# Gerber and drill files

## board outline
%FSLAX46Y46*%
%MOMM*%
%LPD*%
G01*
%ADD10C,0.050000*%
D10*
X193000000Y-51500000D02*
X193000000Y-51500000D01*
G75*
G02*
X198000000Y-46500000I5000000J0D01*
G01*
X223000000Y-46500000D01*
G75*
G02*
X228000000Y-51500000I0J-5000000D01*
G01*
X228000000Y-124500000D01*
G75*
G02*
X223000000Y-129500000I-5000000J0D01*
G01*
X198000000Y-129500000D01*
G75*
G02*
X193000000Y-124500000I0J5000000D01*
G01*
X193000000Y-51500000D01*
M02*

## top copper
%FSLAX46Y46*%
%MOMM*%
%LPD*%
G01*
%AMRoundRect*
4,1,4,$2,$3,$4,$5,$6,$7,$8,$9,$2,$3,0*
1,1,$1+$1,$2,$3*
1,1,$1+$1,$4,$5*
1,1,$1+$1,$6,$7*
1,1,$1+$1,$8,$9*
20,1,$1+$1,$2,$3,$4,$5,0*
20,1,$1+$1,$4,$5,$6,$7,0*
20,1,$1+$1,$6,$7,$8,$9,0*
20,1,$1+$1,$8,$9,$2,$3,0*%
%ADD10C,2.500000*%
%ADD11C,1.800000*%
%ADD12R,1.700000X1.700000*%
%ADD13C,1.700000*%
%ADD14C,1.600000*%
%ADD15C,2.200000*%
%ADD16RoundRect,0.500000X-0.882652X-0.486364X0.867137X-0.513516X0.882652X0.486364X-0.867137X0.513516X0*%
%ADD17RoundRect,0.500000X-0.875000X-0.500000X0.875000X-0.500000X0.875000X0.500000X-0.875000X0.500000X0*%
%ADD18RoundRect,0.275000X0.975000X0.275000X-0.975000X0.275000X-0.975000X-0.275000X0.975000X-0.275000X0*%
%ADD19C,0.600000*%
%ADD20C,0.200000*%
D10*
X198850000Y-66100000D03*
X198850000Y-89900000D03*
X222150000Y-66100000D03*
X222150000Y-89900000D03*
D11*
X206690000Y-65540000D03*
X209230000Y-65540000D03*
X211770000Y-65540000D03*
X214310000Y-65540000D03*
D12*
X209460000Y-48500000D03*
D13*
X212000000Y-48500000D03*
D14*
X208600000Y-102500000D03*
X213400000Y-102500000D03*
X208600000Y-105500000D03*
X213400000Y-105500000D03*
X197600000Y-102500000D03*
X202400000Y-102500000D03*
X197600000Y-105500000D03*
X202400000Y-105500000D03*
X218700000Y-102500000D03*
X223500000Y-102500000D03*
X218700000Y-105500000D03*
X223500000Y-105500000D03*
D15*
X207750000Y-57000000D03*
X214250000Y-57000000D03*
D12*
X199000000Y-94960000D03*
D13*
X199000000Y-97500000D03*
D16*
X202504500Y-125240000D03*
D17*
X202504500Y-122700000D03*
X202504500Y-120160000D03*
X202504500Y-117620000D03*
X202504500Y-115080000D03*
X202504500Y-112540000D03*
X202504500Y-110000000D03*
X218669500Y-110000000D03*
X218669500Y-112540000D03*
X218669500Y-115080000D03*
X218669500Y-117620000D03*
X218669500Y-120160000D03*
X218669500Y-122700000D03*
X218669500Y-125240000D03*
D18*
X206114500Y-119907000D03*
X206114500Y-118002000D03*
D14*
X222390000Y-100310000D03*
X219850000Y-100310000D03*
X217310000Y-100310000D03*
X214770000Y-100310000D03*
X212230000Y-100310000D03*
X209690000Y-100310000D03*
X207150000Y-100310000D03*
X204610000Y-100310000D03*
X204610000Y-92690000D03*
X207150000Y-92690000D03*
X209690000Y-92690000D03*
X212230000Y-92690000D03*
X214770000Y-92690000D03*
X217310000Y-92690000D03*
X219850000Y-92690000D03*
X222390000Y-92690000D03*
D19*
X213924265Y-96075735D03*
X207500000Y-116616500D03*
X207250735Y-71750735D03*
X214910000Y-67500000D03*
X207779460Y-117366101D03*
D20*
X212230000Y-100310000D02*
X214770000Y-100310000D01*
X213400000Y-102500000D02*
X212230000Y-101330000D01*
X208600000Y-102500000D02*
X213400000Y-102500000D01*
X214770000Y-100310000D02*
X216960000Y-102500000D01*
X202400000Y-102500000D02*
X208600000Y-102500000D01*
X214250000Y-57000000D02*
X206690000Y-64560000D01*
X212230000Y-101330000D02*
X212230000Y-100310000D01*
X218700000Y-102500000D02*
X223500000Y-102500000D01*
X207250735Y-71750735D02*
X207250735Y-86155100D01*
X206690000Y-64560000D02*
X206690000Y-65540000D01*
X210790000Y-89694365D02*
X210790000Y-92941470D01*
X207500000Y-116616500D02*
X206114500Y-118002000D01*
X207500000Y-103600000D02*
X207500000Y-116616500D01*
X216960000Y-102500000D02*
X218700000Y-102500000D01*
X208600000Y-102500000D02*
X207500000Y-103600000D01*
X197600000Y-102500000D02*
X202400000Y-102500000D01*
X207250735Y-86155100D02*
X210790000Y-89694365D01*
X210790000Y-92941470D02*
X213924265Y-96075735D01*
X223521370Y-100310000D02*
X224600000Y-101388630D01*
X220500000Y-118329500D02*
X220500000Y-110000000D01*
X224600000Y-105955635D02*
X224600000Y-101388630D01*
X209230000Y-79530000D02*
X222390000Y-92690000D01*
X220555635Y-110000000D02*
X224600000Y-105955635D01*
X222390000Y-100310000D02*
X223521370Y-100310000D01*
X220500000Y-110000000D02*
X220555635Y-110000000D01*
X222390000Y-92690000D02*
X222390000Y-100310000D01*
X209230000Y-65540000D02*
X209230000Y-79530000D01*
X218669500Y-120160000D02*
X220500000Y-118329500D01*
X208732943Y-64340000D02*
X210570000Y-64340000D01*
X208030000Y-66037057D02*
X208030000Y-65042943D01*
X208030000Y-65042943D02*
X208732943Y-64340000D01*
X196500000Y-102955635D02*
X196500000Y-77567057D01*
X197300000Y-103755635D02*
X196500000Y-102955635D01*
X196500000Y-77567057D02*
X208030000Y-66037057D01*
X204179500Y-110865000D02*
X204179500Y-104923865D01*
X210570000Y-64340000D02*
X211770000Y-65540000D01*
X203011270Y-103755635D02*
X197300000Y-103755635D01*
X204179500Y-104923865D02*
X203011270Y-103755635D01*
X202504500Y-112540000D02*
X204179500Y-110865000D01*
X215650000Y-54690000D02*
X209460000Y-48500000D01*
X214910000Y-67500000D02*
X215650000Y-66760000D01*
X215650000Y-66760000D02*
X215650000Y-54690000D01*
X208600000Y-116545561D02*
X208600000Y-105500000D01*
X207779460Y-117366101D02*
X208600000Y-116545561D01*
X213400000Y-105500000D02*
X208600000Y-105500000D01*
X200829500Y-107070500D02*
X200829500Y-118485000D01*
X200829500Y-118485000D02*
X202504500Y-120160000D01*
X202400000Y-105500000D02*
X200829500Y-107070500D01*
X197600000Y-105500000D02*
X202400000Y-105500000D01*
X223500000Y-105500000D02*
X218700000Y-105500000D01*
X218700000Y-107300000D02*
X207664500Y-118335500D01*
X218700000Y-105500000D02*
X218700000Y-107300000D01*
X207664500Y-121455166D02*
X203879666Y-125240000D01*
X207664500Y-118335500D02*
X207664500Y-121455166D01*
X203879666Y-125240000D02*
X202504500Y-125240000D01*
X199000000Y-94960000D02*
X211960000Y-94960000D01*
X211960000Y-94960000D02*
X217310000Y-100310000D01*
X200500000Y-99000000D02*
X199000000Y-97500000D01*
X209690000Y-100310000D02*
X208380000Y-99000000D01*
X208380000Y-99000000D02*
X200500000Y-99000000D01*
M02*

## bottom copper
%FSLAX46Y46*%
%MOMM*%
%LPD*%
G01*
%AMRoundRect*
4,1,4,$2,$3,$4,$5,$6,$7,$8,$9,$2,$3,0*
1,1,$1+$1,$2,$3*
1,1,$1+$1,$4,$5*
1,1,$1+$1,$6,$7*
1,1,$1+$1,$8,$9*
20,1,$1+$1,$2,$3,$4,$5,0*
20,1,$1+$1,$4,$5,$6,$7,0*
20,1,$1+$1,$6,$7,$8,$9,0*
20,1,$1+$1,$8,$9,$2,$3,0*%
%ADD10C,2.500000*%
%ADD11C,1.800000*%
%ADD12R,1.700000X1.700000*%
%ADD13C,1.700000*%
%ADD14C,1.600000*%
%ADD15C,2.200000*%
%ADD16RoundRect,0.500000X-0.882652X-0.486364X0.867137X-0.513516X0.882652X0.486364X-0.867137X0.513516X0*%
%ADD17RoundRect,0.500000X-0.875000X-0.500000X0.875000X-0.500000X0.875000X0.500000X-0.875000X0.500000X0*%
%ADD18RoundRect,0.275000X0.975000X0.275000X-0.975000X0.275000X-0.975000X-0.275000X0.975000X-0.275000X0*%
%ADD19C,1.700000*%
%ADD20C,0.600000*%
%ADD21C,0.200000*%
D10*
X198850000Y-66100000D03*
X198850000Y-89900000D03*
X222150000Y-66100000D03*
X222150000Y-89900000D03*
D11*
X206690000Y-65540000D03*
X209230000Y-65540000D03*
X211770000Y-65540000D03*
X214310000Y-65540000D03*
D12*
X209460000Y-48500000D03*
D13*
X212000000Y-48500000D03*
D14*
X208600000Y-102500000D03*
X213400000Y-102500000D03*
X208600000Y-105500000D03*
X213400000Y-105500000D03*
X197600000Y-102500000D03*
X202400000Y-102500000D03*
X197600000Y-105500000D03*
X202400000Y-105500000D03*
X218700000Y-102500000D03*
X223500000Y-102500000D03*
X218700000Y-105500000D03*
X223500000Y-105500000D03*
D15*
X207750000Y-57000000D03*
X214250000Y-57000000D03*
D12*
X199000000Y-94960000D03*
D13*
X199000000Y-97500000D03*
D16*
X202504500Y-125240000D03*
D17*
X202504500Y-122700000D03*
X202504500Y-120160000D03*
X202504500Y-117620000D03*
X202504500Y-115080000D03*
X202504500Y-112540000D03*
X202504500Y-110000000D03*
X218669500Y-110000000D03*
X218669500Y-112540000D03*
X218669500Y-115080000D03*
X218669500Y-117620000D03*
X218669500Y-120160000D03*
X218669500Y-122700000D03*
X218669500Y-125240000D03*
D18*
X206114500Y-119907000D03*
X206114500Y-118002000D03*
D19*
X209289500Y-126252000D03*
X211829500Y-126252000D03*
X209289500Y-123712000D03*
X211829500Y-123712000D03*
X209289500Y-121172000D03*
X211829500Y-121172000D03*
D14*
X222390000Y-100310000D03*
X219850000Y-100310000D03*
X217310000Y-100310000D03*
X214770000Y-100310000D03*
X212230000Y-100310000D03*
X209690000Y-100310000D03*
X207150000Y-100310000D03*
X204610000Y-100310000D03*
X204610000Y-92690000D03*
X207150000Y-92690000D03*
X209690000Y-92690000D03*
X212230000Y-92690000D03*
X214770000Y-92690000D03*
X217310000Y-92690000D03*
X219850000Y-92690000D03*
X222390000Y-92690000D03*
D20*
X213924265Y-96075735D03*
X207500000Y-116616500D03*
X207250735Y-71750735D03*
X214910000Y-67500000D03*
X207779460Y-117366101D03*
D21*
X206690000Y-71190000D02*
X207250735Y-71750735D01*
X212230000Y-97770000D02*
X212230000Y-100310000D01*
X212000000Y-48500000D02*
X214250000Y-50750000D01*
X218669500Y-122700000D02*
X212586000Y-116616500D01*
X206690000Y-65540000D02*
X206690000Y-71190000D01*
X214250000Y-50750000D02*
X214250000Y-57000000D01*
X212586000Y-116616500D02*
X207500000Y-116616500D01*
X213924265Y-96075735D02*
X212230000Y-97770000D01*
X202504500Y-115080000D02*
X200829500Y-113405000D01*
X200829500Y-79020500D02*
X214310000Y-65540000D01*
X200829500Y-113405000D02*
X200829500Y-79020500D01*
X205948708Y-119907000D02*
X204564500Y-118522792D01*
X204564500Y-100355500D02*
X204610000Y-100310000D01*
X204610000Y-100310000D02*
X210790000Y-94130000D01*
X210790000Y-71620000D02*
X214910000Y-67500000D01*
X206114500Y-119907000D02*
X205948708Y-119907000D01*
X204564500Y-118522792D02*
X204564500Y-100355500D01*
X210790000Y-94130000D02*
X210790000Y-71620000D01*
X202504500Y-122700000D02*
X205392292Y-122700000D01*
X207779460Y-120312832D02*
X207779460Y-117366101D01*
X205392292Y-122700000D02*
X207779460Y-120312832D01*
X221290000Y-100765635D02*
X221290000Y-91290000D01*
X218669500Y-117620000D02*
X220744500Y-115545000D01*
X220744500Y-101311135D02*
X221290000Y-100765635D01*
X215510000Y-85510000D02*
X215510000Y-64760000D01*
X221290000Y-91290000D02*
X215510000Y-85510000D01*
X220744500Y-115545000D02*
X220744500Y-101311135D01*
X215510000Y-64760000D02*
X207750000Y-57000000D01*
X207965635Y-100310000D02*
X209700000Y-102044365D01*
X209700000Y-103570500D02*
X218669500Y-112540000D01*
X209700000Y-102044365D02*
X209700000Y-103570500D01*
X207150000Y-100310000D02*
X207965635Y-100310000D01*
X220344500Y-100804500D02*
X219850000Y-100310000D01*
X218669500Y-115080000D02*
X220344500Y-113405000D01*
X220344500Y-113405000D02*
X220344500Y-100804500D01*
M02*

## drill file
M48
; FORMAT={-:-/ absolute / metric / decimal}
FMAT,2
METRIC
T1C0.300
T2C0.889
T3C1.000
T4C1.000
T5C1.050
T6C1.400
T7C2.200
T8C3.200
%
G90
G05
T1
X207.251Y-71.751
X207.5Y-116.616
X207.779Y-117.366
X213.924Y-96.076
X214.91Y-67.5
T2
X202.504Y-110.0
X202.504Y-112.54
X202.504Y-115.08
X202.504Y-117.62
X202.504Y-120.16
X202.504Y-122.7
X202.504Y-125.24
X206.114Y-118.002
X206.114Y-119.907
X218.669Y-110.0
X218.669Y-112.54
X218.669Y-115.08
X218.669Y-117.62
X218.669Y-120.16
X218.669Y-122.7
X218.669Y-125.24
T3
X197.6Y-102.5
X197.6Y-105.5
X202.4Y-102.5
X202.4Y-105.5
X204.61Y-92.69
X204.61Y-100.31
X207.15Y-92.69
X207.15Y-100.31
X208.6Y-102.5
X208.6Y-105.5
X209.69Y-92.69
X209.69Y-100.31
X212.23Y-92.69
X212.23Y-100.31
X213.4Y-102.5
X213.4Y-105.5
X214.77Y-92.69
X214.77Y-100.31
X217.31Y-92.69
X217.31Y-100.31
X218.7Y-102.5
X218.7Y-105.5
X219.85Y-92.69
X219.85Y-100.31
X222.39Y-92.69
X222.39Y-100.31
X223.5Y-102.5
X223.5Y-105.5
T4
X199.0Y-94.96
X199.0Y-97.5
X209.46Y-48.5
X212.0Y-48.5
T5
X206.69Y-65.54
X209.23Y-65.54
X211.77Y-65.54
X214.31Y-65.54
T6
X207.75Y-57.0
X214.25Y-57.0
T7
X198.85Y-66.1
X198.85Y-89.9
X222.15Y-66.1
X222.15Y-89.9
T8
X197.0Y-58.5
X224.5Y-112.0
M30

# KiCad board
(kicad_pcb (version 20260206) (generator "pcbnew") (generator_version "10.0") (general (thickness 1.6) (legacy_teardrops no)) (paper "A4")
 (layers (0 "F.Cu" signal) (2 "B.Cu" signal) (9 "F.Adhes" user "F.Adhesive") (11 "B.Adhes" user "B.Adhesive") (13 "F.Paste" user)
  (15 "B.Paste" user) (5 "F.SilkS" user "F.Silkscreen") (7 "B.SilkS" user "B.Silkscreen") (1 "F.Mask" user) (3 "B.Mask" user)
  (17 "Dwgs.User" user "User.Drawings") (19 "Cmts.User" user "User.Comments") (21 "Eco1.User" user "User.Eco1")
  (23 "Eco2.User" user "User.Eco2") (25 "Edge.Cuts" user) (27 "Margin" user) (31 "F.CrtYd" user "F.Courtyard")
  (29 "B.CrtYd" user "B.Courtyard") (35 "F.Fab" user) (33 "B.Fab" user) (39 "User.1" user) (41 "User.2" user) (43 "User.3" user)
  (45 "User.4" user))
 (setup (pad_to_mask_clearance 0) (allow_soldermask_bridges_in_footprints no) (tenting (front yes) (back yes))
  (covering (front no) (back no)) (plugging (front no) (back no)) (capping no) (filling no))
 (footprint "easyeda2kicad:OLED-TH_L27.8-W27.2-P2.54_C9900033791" (layer "F.Cu") (at 210.5 65.54)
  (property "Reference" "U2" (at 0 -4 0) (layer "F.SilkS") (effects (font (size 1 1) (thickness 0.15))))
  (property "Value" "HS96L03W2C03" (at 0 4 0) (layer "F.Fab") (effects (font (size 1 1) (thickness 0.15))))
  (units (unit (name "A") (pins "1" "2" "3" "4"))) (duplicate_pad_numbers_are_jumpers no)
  (pad "" thru_hole circle (at -11.65 0.56) (size 2.5 2.5) (drill 2.2) (layers "*.Cu" "*.Mask") (remove_unused_layers no))
  (pad "" thru_hole circle (at -11.65 24.36) (size 2.5 2.5) (drill 2.2) (layers "*.Cu" "*.Mask") (remove_unused_layers no))
  (pad "" thru_hole circle (at 11.65 0.56) (size 2.5 2.5) (drill 2.2) (layers "*.Cu" "*.Mask") (remove_unused_layers no))
  (pad "" thru_hole circle (at 11.65 24.36) (size 2.5 2.5) (drill 2.2) (layers "*.Cu" "*.Mask") (remove_unused_layers no))
  (pad "1" thru_hole circle (at -3.81 0) (size 1.8 1.8) (drill 1.049986) (layers "*.Cu" "*.Mask") (remove_unused_layers no) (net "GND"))
  (pad "2" thru_hole circle (at -1.27 0) (size 1.8 1.8) (drill 1.049986) (layers "*.Cu" "*.Mask") (remove_unused_layers no) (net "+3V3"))
  (pad "3" thru_hole circle (at 1.27 0) (size 1.8 1.8) (drill 1.049986) (layers "*.Cu" "*.Mask") (remove_unused_layers no)
   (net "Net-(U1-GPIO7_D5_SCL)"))
  (pad "4" thru_hole circle (at 3.81 0) (size 1.8 1.8) (drill 1.049986) (layers "*.Cu" "*.Mask") (remove_unused_layers no)
   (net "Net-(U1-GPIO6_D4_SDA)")))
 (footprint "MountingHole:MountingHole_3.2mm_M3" (layer "F.Cu") (at 224.5 112)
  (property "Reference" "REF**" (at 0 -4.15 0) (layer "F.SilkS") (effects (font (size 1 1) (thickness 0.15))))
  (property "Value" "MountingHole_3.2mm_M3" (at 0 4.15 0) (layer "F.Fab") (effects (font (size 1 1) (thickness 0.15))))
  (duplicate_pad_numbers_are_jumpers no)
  (pad "" np_thru_hole circle (at 0 0) (size 3.2 3.2) (drill 3.2) (layers "*.Cu" "*.Mask")))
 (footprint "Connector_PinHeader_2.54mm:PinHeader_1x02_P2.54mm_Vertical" (layer "F.Cu") (at 209.46 48.5 90)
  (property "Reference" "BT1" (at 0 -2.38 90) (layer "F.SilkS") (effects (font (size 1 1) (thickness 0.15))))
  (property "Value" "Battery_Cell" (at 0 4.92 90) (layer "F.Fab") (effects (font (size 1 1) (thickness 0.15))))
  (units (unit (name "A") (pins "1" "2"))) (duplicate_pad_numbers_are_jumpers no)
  (pad "1" thru_hole rect (at 0 0 90) (size 1.7 1.7) (drill 1) (layers "*.Cu" "*.Mask") (remove_unused_layers no) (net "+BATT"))
  (pad "2" thru_hole circle (at 0 2.54 90) (size 1.7 1.7) (drill 1) (layers "*.Cu" "*.Mask") (remove_unused_layers no) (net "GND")))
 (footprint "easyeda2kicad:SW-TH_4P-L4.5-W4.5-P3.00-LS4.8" (layer "F.Cu") (at 211 104)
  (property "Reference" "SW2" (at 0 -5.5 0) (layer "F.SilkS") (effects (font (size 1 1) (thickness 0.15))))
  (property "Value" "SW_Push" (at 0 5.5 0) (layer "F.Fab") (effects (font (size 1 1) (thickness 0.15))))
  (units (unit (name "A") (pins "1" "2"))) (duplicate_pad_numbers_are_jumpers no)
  (pad "1" thru_hole circle (at -2.4 -1.5) (size 1.6 1.6) (drill 0.999998) (layers "*.Cu" "*.Mask") (remove_unused_layers no) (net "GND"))
  (pad "1" thru_hole circle (at 2.4 -1.5) (size 1.6 1.6) (drill 0.999998) (layers "*.Cu" "*.Mask") (remove_unused_layers no) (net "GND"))
  (pad "2" thru_hole circle (at -2.4 1.5) (size 1.6 1.6) (drill 0.999998) (layers "*.Cu" "*.Mask") (remove_unused_layers no)
   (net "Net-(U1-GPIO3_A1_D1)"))
  (pad "2" thru_hole circle (at 2.4 1.5) (size 1.6 1.6) (drill 0.999998) (layers "*.Cu" "*.Mask") (remove_unused_layers no)
   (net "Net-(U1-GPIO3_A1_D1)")))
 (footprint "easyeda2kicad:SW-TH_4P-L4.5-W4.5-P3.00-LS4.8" (layer "F.Cu") (at 200 104)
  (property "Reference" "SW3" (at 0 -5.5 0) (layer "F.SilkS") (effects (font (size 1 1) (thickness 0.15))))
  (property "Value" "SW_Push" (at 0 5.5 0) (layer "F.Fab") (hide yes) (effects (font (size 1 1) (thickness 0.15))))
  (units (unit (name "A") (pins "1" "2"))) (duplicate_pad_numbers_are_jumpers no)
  (pad "1" thru_hole circle (at -2.4 -1.5) (size 1.6 1.6) (drill 0.999998) (layers "*.Cu" "*.Mask") (remove_unused_layers no) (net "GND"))
  (pad "1" thru_hole circle (at 2.4 -1.5) (size 1.6 1.6) (drill 0.999998) (layers "*.Cu" "*.Mask") (remove_unused_layers no) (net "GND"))
  (pad "2" thru_hole circle (at -2.4 1.5) (size 1.6 1.6) (drill 0.999998) (layers "*.Cu" "*.Mask") (remove_unused_layers no)
   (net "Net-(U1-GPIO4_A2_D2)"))
  (pad "2" thru_hole circle (at 2.4 1.5) (size 1.6 1.6) (drill 0.999998) (layers "*.Cu" "*.Mask") (remove_unused_layers no)
   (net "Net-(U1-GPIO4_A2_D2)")))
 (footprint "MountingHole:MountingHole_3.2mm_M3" (layer "F.Cu") (at 197 58.5)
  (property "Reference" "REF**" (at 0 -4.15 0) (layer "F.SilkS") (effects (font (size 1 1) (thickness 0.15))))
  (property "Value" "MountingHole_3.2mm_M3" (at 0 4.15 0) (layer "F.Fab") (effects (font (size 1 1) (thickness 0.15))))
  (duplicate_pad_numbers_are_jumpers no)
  (pad "" np_thru_hole circle (at 0 0) (size 3.2 3.2) (drill 3.2) (layers "*.Cu" "*.Mask")))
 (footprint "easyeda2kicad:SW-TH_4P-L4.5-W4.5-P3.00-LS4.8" (layer "F.Cu") (at 221.1 104)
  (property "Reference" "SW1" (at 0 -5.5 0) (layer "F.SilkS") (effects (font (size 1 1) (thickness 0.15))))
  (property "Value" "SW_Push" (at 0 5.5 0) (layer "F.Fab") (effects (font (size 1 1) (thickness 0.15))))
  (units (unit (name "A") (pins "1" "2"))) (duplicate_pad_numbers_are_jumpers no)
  (pad "1" thru_hole circle (at -2.4 -1.5) (size 1.6 1.6) (drill 0.999998) (layers "*.Cu" "*.Mask") (remove_unused_layers no) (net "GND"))
  (pad "1" thru_hole circle (at 2.4 -1.5) (size 1.6 1.6) (drill 0.999998) (layers "*.Cu" "*.Mask") (remove_unused_layers no) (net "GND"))
  (pad "2" thru_hole circle (at -2.4 1.5) (size 1.6 1.6) (drill 0.999998) (layers "*.Cu" "*.Mask") (remove_unused_layers no)
   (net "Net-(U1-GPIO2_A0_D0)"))
  (pad "2" thru_hole circle (at 2.4 1.5) (size 1.6 1.6) (drill 0.999998) (layers "*.Cu" "*.Mask") (remove_unused_layers no)
   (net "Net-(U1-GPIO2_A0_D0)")))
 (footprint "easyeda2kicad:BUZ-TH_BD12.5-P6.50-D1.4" (layer "F.Cu") (at 211 57)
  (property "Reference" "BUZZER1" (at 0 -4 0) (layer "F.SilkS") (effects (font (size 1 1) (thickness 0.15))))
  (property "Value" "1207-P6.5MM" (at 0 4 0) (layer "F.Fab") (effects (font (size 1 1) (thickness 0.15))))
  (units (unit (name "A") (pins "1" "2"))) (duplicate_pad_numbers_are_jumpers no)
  (pad "1" thru_hole circle (at -3.25 0) (size 2.2 2.2) (drill 1.399998) (layers "*.Cu" "*.Mask") (remove_unused_layers no)
   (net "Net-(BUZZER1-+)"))
  (pad "2" thru_hole circle (at 3.25 0) (size 2.2 2.2) (drill 1.399998) (layers "*.Cu" "*.Mask") (remove_unused_layers no) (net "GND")))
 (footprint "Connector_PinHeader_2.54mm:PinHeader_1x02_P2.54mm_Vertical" (layer "F.Cu") (at 199 94.96)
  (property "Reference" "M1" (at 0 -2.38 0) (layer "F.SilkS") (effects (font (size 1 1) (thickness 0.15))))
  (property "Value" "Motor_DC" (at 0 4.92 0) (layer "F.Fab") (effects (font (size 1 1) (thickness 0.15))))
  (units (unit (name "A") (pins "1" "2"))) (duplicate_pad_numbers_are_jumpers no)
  (pad "1" thru_hole rect (at 0 0) (size 1.7 1.7) (drill 1) (layers "*.Cu" "*.Mask") (remove_unused_layers no) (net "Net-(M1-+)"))
  (pad "2" thru_hole circle (at 0 2.54) (size 1.7 1.7) (drill 1) (layers "*.Cu" "*.Mask") (remove_unused_layers no) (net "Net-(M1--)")))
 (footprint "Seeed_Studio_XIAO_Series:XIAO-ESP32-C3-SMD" (layer "B.Cu") (at 201.6695 107.12)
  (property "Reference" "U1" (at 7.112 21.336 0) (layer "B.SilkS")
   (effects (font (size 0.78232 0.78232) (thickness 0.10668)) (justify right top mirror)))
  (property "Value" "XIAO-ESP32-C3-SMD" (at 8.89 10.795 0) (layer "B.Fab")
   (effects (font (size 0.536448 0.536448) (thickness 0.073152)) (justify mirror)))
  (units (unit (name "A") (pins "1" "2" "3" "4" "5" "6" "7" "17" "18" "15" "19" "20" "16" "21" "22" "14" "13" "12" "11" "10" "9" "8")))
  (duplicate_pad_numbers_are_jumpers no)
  (pad "1" thru_hole roundrect (at 0.835 18.12 359.111) (size 2.75 2) (drill 0.889) (layers "*.Cu" "*.Mask") (remove_unused_layers no)
   (roundrect_rratio 0.25) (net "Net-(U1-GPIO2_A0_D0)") (solder_mask_margin 0.0508) (thermal_bridge_angle 45))
  (pad "2" thru_hole roundrect (at 0.835 15.58) (size 2.75 2) (drill 0.889) (layers "*.Cu" "*.Mask") (remove_unused_layers no)
   (roundrect_rratio 0.25) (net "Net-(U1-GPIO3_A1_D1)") (solder_mask_margin 0.0508) (thermal_bridge_angle 45))
  (pad "3" thru_hole roundrect (at 0.835 13.04) (size 2.75 2) (drill 0.889) (layers "*.Cu" "*.Mask") (remove_unused_layers no)
   (roundrect_rratio 0.25) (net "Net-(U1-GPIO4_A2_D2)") (solder_mask_margin 0.0508) (thermal_bridge_angle 45))
  (pad "4" thru_hole roundrect (at 0.835 10.5) (size 2.75 2) (drill 0.889) (layers "*.Cu" "*.Mask") (remove_unused_layers no)
   (roundrect_rratio 0.25) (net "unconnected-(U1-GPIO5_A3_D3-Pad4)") (solder_mask_margin 0.0508) (thermal_bridge_angle 45))
  (pad "5" thru_hole roundrect (at 0.835 7.96) (size 2.75 2) (drill 0.889) (layers "*.Cu" "*.Mask") (remove_unused_layers no)
   (roundrect_rratio 0.25) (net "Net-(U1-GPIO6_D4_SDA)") (solder_mask_margin 0.0508) (thermal_bridge_angle 45))
  (pad "6" thru_hole roundrect (at 0.835 5.42) (size 2.75 2) (drill 0.889) (layers "*.Cu" "*.Mask") (remove_unused_layers no)
   (roundrect_rratio 0.25) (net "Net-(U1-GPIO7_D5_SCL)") (solder_mask_margin 0.0508) (thermal_bridge_angle 45))
  (pad "7" thru_hole roundrect (at 0.835 2.88) (size 2.75 2) (drill 0.889) (layers "*.Cu" "*.Mask") (remove_unused_layers no)
   (roundrect_rratio 0.25) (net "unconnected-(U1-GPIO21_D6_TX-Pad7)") (solder_mask_margin 0.0508) (thermal_bridge_angle 45))
  (pad "8" thru_hole roundrect (at 17 2.88) (size 2.75 2) (drill 0.889) (layers "*.Cu" "*.Mask") (remove_unused_layers no)
   (roundrect_rratio 0.25) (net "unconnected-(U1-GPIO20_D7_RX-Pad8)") (solder_mask_margin 0.0508) (thermal_bridge_angle 45))
  (pad "9" thru_hole roundrect (at 17 5.42) (size 2.75 2) (drill 0.889) (layers "*.Cu" "*.Mask") (remove_unused_layers no)
   (roundrect_rratio 0.25) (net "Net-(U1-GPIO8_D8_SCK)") (solder_mask_margin 0.0508) (thermal_bridge_angle 45))
  (pad "10" thru_hole roundrect (at 17 7.96) (size 2.75 2) (drill 0.889) (layers "*.Cu" "*.Mask") (remove_unused_layers no)
   (roundrect_rratio 0.25) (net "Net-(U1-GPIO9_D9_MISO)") (solder_mask_margin 0.0508) (thermal_bridge_angle 45))
  (pad "11" thru_hole roundrect (at 17 10.5) (size 2.75 2) (drill 0.889) (layers "*.Cu" "*.Mask") (remove_unused_layers no)
   (roundrect_rratio 0.25) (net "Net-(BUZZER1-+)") (solder_mask_margin 0.0508) (thermal_bridge_angle 45))
  (pad "12" thru_hole roundrect (at 17 13.04) (size 2.75 2) (drill 0.889) (layers "*.Cu" "*.Mask") (remove_unused_layers no)
   (roundrect_rratio 0.25) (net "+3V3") (solder_mask_margin 0.0508) (thermal_bridge_angle 45))
  (pad "13" thru_hole roundrect (at 17 15.58) (size 2.75 2) (drill 0.889) (layers "*.Cu" "*.Mask") (remove_unused_layers no)
   (roundrect_rratio 0.25) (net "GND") (solder_mask_margin 0.0508) (thermal_bridge_angle 45))
  (pad "14" thru_hole roundrect (at 17 18.12) (size 2.75 2) (drill 0.889) (layers "*.Cu" "*.Mask") (remove_unused_layers no)
   (roundrect_rratio 0.25) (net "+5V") (solder_mask_margin 0.0508) (thermal_bridge_angle 45))
  (pad "15" thru_hole roundrect (at 4.445 12.787 180) (size 2.5 1.1) (drill 0.889) (layers "*.Cu" "*.Mask") (remove_unused_layers no)
   (roundrect_rratio 0.25) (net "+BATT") (thermal_bridge_angle 45))
  (pad "16" thru_hole roundrect (at 4.445 10.882 180) (size 2.5 1.1) (drill 0.889) (layers "*.Cu" "*.Mask") (remove_unused_layers no)
   (roundrect_rratio 0.25) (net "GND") (thermal_bridge_angle 45))
  (pad "17" smd circle (at 7.62 19.132) (size 1.7 1.7) (layers "B.Cu" "B.Mask" "B.Paste") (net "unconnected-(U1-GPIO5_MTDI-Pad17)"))
  (pad "18" smd circle (at 10.16 19.132) (size 1.7 1.7) (layers "B.Cu" "B.Mask" "B.Paste") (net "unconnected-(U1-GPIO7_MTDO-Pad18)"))
  (pad "19" smd circle (at 7.62 16.592) (size 1.7 1.7) (layers "B.Cu" "B.Mask" "B.Paste") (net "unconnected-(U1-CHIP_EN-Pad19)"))
  (pad "20" smd circle (at 10.16 16.592) (size 1.7 1.7) (layers "B.Cu" "B.Mask" "B.Paste") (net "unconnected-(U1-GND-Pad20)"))
  (pad "21" smd circle (at 7.62 14.052) (size 1.7 1.7) (layers "B.Cu" "B.Mask" "B.Paste") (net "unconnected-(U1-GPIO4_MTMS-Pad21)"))
  (pad "22" smd circle (at 10.16 14.052) (size 1.7 1.7) (layers "B.Cu" "B.Mask" "B.Paste") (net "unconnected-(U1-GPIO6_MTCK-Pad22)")))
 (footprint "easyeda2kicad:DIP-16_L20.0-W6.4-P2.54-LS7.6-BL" (layer "B.Cu") (at 213.5 96.5 180)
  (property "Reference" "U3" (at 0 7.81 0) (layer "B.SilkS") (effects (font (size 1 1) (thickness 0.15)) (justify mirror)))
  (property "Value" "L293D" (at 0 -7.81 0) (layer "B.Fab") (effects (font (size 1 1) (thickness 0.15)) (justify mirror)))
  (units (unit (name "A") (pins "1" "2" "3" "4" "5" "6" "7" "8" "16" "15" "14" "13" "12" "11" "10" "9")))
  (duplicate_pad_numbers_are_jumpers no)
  (pad "1" thru_hole circle (at -8.89 -3.81 90) (size 1.6 1.6) (drill 0.999998) (layers "*.Cu" "*.Mask") (remove_unused_layers no)
   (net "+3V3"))
  (pad "2" thru_hole circle (at -6.35 -3.81 90) (size 1.6 1.6) (drill 0.999998) (layers "*.Cu" "*.Mask") (remove_unused_layers no)
   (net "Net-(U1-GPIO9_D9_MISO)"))
  (pad "3" thru_hole circle (at -3.81 -3.81 90) (size 1.6 1.6) (drill 0.999998) (layers "*.Cu" "*.Mask") (remove_unused_layers no)
   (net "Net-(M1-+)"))
  (pad "4" thru_hole circle (at -1.27 -3.81 90) (size 1.6 1.6) (drill 0.999998) (layers "*.Cu" "*.Mask") (remove_unused_layers no)
   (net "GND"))
  (pad "5" thru_hole circle (at 1.27 -3.81 90) (size 1.6 1.6) (drill 0.999998) (layers "*.Cu" "*.Mask") (remove_unused_layers no)
   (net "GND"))
  (pad "6" thru_hole circle (at 3.81 -3.81 90) (size 1.6 1.6) (drill 0.999998) (layers "*.Cu" "*.Mask") (remove_unused_layers no)
   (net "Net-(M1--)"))
  (pad "7" thru_hole circle (at 6.35 -3.81 90) (size 1.6 1.6) (drill 0.999998) (layers "*.Cu" "*.Mask") (remove_unused_layers no)
   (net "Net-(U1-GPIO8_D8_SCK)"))
  (pad "8" thru_hole circle (at 8.89 -3.81 90) (size 1.6 1.6) (drill 0.999998) (layers "*.Cu" "*.Mask") (remove_unused_layers no)
   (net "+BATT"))
  (pad "9" thru_hole circle (at 8.89 3.81 90) (size 1.6 1.6) (drill 0.999998) (layers "*.Cu" "*.Mask") (remove_unused_layers no)
   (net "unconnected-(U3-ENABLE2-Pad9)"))
  (pad "10" thru_hole circle (at 6.35 3.81 90) (size 1.6 1.6) (drill 0.999998) (layers "*.Cu" "*.Mask") (remove_unused_layers no)
   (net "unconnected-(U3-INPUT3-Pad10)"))
  (pad "11" thru_hole circle (at 3.81 3.81 90) (size 1.6 1.6) (drill 0.999998) (layers "*.Cu" "*.Mask") (remove_unused_layers no)
   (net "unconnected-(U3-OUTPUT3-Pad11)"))
  (pad "12" thru_hole circle (at 1.27 3.81 90) (size 1.6 1.6) (drill 0.999998) (layers "*.Cu" "*.Mask") (remove_unused_layers no)
   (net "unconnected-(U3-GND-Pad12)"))
  (pad "13" thru_hole circle (at -1.27 3.81 90) (size 1.6 1.6) (drill 0.999998) (layers "*.Cu" "*.Mask") (remove_unused_layers no)
   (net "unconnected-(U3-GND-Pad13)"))
  (pad "14" thru_hole circle (at -3.81 3.81 90) (size 1.6 1.6) (drill 0.999998) (layers "*.Cu" "*.Mask") (remove_unused_layers no)
   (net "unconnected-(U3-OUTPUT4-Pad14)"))
  (pad "15" thru_hole circle (at -6.35 3.81 90) (size 1.6 1.6) (drill 0.999998) (layers "*.Cu" "*.Mask") (remove_unused_layers no)
   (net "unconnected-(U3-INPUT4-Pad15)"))
  (pad "16" thru_hole circle (at -8.89 3.81 90) (size 1.6 1.6) (drill 0.999998) (layers "*.Cu" "*.Mask") (remove_unused_layers no)
   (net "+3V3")))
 (gr_rect (start 193 46.5) (end 228 129.5) (radius 5) (stroke (width 0.05) (type solid)) (fill no) (layer "Edge.Cuts"))
 (segment (start 212.23 100.31) (end 214.77 100.31) (width 0.2) (layer "F.Cu") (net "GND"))
 (segment (start 213.4 102.5) (end 212.23 101.33) (width 0.2) (layer "F.Cu") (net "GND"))
 (segment (start 208.6 102.5) (end 213.4 102.5) (width 0.2) (layer "F.Cu") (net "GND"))
 (segment (start 214.77 100.31) (end 216.96 102.5) (width 0.2) (layer "F.Cu") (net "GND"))
 (segment (start 202.4 102.5) (end 208.6 102.5) (width 0.2) (layer "F.Cu") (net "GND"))
 (segment (start 214.25 57) (end 206.69 64.56) (width 0.2) (layer "F.Cu") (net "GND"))
 (segment (start 212.23 101.33) (end 212.23 100.31) (width 0.2) (layer "F.Cu") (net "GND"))
 (segment (start 218.7 102.5) (end 223.5 102.5) (width 0.2) (layer "F.Cu") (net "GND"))
 (segment (start 207.250735 71.750735) (end 207.250735 86.1551) (width 0.2) (layer "F.Cu") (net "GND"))
 (segment (start 206.69 64.56) (end 206.69 65.54) (width 0.2) (layer "F.Cu") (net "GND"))
 (segment (start 210.79 89.694365) (end 210.79 92.94147) (width 0.2) (layer "F.Cu") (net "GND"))
 (segment (start 207.5 116.6165) (end 206.1145 118.002) (width 0.2) (layer "F.Cu") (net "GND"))
 (segment (start 207.5 103.6) (end 207.5 116.6165) (width 0.2) (layer "F.Cu") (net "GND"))
 (segment (start 216.96 102.5) (end 218.7 102.5) (width 0.2) (layer "F.Cu") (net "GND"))
 (segment (start 208.6 102.5) (end 207.5 103.6) (width 0.2) (layer "F.Cu") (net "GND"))
 (segment (start 197.6 102.5) (end 202.4 102.5) (width 0.2) (layer "F.Cu") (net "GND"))
 (segment (start 207.250735 86.1551) (end 210.79 89.694365) (width 0.2) (layer "F.Cu") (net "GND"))
 (segment (start 210.79 92.94147) (end 213.924265 96.075735) (width 0.2) (layer "F.Cu") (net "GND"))
 (via (at 213.924265 96.075735) (size 0.6) (drill 0.3) (layers "F.Cu" "B.Cu") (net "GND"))
 (via (at 207.5 116.6165) (size 0.6) (drill 0.3) (layers "F.Cu" "B.Cu") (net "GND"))
 (via (at 207.250735 71.750735) (size 0.6) (drill 0.3) (layers "F.Cu" "B.Cu") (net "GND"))
 (segment (start 206.69 71.19) (end 207.250735 71.750735) (width 0.2) (layer "B.Cu") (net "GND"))
 (segment (start 212.23 97.77) (end 212.23 100.31) (width 0.2) (layer "B.Cu") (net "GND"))
 (segment (start 212 48.5) (end 214.25 50.75) (width 0.2) (layer "B.Cu") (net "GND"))
 (segment (start 218.6695 122.7) (end 212.586 116.6165) (width 0.2) (layer "B.Cu") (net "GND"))
 (segment (start 206.69 65.54) (end 206.69 71.19) (width 0.2) (layer "B.Cu") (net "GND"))
 (segment (start 214.25 50.75) (end 214.25 57) (width 0.2) (layer "B.Cu") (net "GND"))
 (segment (start 212.586 116.6165) (end 207.5 116.6165) (width 0.2) (layer "B.Cu") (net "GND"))
 (segment (start 213.924265 96.075735) (end 212.23 97.77) (width 0.2) (layer "B.Cu") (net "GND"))
 (segment (start 223.52137 100.31) (end 224.6 101.38863) (width 0.2) (layer "F.Cu") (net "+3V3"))
 (segment (start 220.5 118.3295) (end 220.5 110) (width 0.2) (layer "F.Cu") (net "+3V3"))
 (segment (start 224.6 105.955635) (end 224.6 101.38863) (width 0.2) (layer "F.Cu") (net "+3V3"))
 (segment (start 209.23 79.53) (end 222.39 92.69) (width 0.2) (layer "F.Cu") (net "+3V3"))
 (segment (start 220.555635 110) (end 224.6 105.955635) (width 0.2) (layer "F.Cu") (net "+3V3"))
 (segment (start 222.39 100.31) (end 223.52137 100.31) (width 0.2) (layer "F.Cu") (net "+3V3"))
 (segment (start 220.5 110) (end 220.555635 110) (width 0.2) (layer "F.Cu") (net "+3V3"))
 (segment (start 222.39 92.69) (end 222.39 100.31) (width 0.2) (layer "F.Cu") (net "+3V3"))
 (segment (start 209.23 65.54) (end 209.23 79.53) (width 0.2) (layer "F.Cu") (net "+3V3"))
 (segment (start 218.6695 120.16) (end 220.5 118.3295) (width 0.2) (layer "F.Cu") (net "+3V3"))
 (segment (start 208.732943 64.34) (end 210.57 64.34) (width 0.2) (layer "F.Cu") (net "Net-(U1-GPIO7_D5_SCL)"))
 (segment (start 208.03 66.037057) (end 208.03 65.042943) (width 0.2) (layer "F.Cu") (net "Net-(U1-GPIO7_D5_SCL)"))
 (segment (start 208.03 65.042943) (end 208.732943 64.34) (width 0.2) (layer "F.Cu") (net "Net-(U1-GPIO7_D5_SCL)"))
 (segment (start 196.5 102.955635) (end 196.5 77.567057) (width 0.2) (layer "F.Cu") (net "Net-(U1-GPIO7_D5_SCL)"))
 (segment (start 197.3 103.755635) (end 196.5 102.955635) (width 0.2) (layer "F.Cu") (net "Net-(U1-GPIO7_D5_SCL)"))
 (segment (start 196.5 77.567057) (end 208.03 66.037057) (width 0.2) (layer "F.Cu") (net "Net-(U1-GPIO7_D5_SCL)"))
 (segment (start 204.1795 110.865) (end 204.1795 104.923865) (width 0.2) (layer "F.Cu") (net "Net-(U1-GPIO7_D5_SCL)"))
 (segment (start 210.57 64.34) (end 211.77 65.54) (width 0.2) (layer "F.Cu") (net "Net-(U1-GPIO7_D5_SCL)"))
 (segment (start 203.01127 103.755635) (end 197.3 103.755635) (width 0.2) (layer "F.Cu") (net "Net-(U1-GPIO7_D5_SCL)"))
 (segment (start 204.1795 104.923865) (end 203.01127 103.755635) (width 0.2) (layer "F.Cu") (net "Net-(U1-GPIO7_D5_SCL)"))
 (segment (start 202.5045 112.54) (end 204.1795 110.865) (width 0.2) (layer "F.Cu") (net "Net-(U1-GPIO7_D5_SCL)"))
 (segment (start 202.5045 115.08) (end 200.8295 113.405) (width 0.2) (layer "B.Cu") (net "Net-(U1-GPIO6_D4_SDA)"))
 (segment (start 200.8295 79.0205) (end 214.31 65.54) (width 0.2) (layer "B.Cu") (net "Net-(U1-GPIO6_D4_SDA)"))
 (segment (start 200.8295 113.405) (end 200.8295 79.0205) (width 0.2) (layer "B.Cu") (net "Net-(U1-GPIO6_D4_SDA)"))
 (segment (start 215.65 54.69) (end 209.46 48.5) (width 0.2) (layer "F.Cu") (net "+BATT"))
 (segment (start 214.91 67.5) (end 215.65 66.76) (width 0.2) (layer "F.Cu") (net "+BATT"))
 (segment (start 215.65 66.76) (end 215.65 54.69) (width 0.2) (layer "F.Cu") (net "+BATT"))
 (via (at 214.91 67.5) (size 0.6) (drill 0.3) (layers "F.Cu" "B.Cu") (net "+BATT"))
 (segment (start 205.948708 119.907) (end 204.5645 118.522792) (width 0.2) (layer "B.Cu") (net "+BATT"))
 (segment (start 204.5645 100.3555) (end 204.61 100.31) (width 0.2) (layer "B.Cu") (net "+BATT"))
 (segment (start 204.61 100.31) (end 210.79 94.13) (width 0.2) (layer "B.Cu") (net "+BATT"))
 (segment (start 210.79 71.62) (end 214.91 67.5) (width 0.2) (layer "B.Cu") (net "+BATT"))
 (segment (start 206.1145 119.907) (end 205.948708 119.907) (width 0.2) (layer "B.Cu") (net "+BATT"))
 (segment (start 204.5645 118.522792) (end 204.5645 100.3555) (width 0.2) (layer "B.Cu") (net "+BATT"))
 (segment (start 210.79 94.13) (end 210.79 71.62) (width 0.2) (layer "B.Cu") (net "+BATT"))
 (segment (start 208.6 116.545561) (end 208.6 105.5) (width 0.2) (layer "F.Cu") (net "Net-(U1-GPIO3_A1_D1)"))
 (segment (start 207.77946 117.366101) (end 208.6 116.545561) (width 0.2) (layer "F.Cu") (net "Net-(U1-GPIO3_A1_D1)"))
 (segment (start 213.4 105.5) (end 208.6 105.5) (width 0.2) (layer "F.Cu") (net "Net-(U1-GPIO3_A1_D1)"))
 (via (at 207.77946 117.366101) (size 0.6) (drill 0.3) (layers "F.Cu" "B.Cu") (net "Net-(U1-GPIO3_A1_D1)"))
 (segment (start 202.5045 122.7) (end 205.392292 122.7) (width 0.2) (layer "B.Cu") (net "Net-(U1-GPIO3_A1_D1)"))
 (segment (start 207.77946 120.312832) (end 207.77946 117.366101) (width 0.2) (layer "B.Cu") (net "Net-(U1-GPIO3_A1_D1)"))
 (segment (start 205.392292 122.7) (end 207.77946 120.312832) (width 0.2) (layer "B.Cu") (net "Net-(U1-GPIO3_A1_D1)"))
 (segment (start 200.8295 107.0705) (end 200.8295 118.485) (width 0.2) (layer "F.Cu") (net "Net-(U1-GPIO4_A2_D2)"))
 (segment (start 200.8295 118.485) (end 202.5045 120.16) (width 0.2) (layer "F.Cu") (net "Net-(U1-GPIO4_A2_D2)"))
 (segment (start 202.4 105.5) (end 200.8295 107.0705) (width 0.2) (layer "F.Cu") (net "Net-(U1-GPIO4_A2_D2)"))
 (segment (start 197.6 105.5) (end 202.4 105.5) (width 0.2) (layer "F.Cu") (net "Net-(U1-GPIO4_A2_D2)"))
 (segment (start 223.5 105.5) (end 218.7 105.5) (width 0.2) (layer "F.Cu") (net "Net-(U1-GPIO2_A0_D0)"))
 (segment (start 218.7 107.3) (end 207.6645 118.3355) (width 0.2) (layer "F.Cu") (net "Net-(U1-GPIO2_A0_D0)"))
 (segment (start 218.7 105.5) (end 218.7 107.3) (width 0.2) (layer "F.Cu") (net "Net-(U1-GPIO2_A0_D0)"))
 (segment (start 207.6645 121.455166) (end 203.879666 125.24) (width 0.2) (layer "F.Cu") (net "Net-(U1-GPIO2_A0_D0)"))
 (segment (start 207.6645 118.3355) (end 207.6645 121.455166) (width 0.2) (layer "F.Cu") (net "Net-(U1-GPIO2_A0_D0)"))
 (segment (start 203.879666 125.24) (end 202.5045 125.24) (width 0.2) (layer "F.Cu") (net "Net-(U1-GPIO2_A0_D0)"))
 (segment (start 221.29 100.765635) (end 221.29 91.29) (width 0.2) (layer "B.Cu") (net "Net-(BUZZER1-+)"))
 (segment (start 218.6695 117.62) (end 220.7445 115.545) (width 0.2) (layer "B.Cu") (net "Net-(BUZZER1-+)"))
 (segment (start 220.7445 101.311135) (end 221.29 100.765635) (width 0.2) (layer "B.Cu") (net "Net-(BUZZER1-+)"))
 (segment (start 215.51 85.51) (end 215.51 64.76) (width 0.2) (layer "B.Cu") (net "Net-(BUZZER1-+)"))
 (segment (start 221.29 91.29) (end 215.51 85.51) (width 0.2) (layer "B.Cu") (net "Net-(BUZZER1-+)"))
 (segment (start 220.7445 115.545) (end 220.7445 101.311135) (width 0.2) (layer "B.Cu") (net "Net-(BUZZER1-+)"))
 (segment (start 215.51 64.76) (end 207.75 57) (width 0.2) (layer "B.Cu") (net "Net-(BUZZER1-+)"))
 (segment (start 199 94.96) (end 211.96 94.96) (width 0.2) (layer "F.Cu") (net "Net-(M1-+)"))
 (segment (start 211.96 94.96) (end 217.31 100.31) (width 0.2) (layer "F.Cu") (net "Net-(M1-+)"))
 (segment (start 200.5 99) (end 199 97.5) (width 0.2) (layer "F.Cu") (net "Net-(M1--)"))
 (segment (start 209.69 100.31) (end 208.38 99) (width 0.2) (layer "F.Cu") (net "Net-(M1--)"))
 (segment (start 208.38 99) (end 200.5 99) (width 0.2) (layer "F.Cu") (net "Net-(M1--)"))
 (segment (start 207.965635 100.31) (end 209.7 102.044365) (width 0.2) (layer "B.Cu") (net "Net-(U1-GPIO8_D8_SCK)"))
 (segment (start 209.7 103.5705) (end 218.6695 112.54) (width 0.2) (layer "B.Cu") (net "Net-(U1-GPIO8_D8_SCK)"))
 (segment (start 209.7 102.044365) (end 209.7 103.5705) (width 0.2) (layer "B.Cu") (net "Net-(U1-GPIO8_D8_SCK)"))
 (segment (start 207.15 100.31) (end 207.965635 100.31) (width 0.2) (layer "B.Cu") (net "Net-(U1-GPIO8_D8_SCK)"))
 (segment (start 220.3445 100.8045) (end 219.85 100.31) (width 0.2) (layer "B.Cu") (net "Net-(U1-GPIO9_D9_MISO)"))
 (segment (start 218.6695 115.08) (end 220.3445 113.405) (width 0.2) (layer "B.Cu") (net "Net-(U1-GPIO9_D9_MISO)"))
 (segment (start 220.3445 113.405) (end 220.3445 100.8045) (width 0.2) (layer "B.Cu") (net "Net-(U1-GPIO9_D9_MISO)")))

